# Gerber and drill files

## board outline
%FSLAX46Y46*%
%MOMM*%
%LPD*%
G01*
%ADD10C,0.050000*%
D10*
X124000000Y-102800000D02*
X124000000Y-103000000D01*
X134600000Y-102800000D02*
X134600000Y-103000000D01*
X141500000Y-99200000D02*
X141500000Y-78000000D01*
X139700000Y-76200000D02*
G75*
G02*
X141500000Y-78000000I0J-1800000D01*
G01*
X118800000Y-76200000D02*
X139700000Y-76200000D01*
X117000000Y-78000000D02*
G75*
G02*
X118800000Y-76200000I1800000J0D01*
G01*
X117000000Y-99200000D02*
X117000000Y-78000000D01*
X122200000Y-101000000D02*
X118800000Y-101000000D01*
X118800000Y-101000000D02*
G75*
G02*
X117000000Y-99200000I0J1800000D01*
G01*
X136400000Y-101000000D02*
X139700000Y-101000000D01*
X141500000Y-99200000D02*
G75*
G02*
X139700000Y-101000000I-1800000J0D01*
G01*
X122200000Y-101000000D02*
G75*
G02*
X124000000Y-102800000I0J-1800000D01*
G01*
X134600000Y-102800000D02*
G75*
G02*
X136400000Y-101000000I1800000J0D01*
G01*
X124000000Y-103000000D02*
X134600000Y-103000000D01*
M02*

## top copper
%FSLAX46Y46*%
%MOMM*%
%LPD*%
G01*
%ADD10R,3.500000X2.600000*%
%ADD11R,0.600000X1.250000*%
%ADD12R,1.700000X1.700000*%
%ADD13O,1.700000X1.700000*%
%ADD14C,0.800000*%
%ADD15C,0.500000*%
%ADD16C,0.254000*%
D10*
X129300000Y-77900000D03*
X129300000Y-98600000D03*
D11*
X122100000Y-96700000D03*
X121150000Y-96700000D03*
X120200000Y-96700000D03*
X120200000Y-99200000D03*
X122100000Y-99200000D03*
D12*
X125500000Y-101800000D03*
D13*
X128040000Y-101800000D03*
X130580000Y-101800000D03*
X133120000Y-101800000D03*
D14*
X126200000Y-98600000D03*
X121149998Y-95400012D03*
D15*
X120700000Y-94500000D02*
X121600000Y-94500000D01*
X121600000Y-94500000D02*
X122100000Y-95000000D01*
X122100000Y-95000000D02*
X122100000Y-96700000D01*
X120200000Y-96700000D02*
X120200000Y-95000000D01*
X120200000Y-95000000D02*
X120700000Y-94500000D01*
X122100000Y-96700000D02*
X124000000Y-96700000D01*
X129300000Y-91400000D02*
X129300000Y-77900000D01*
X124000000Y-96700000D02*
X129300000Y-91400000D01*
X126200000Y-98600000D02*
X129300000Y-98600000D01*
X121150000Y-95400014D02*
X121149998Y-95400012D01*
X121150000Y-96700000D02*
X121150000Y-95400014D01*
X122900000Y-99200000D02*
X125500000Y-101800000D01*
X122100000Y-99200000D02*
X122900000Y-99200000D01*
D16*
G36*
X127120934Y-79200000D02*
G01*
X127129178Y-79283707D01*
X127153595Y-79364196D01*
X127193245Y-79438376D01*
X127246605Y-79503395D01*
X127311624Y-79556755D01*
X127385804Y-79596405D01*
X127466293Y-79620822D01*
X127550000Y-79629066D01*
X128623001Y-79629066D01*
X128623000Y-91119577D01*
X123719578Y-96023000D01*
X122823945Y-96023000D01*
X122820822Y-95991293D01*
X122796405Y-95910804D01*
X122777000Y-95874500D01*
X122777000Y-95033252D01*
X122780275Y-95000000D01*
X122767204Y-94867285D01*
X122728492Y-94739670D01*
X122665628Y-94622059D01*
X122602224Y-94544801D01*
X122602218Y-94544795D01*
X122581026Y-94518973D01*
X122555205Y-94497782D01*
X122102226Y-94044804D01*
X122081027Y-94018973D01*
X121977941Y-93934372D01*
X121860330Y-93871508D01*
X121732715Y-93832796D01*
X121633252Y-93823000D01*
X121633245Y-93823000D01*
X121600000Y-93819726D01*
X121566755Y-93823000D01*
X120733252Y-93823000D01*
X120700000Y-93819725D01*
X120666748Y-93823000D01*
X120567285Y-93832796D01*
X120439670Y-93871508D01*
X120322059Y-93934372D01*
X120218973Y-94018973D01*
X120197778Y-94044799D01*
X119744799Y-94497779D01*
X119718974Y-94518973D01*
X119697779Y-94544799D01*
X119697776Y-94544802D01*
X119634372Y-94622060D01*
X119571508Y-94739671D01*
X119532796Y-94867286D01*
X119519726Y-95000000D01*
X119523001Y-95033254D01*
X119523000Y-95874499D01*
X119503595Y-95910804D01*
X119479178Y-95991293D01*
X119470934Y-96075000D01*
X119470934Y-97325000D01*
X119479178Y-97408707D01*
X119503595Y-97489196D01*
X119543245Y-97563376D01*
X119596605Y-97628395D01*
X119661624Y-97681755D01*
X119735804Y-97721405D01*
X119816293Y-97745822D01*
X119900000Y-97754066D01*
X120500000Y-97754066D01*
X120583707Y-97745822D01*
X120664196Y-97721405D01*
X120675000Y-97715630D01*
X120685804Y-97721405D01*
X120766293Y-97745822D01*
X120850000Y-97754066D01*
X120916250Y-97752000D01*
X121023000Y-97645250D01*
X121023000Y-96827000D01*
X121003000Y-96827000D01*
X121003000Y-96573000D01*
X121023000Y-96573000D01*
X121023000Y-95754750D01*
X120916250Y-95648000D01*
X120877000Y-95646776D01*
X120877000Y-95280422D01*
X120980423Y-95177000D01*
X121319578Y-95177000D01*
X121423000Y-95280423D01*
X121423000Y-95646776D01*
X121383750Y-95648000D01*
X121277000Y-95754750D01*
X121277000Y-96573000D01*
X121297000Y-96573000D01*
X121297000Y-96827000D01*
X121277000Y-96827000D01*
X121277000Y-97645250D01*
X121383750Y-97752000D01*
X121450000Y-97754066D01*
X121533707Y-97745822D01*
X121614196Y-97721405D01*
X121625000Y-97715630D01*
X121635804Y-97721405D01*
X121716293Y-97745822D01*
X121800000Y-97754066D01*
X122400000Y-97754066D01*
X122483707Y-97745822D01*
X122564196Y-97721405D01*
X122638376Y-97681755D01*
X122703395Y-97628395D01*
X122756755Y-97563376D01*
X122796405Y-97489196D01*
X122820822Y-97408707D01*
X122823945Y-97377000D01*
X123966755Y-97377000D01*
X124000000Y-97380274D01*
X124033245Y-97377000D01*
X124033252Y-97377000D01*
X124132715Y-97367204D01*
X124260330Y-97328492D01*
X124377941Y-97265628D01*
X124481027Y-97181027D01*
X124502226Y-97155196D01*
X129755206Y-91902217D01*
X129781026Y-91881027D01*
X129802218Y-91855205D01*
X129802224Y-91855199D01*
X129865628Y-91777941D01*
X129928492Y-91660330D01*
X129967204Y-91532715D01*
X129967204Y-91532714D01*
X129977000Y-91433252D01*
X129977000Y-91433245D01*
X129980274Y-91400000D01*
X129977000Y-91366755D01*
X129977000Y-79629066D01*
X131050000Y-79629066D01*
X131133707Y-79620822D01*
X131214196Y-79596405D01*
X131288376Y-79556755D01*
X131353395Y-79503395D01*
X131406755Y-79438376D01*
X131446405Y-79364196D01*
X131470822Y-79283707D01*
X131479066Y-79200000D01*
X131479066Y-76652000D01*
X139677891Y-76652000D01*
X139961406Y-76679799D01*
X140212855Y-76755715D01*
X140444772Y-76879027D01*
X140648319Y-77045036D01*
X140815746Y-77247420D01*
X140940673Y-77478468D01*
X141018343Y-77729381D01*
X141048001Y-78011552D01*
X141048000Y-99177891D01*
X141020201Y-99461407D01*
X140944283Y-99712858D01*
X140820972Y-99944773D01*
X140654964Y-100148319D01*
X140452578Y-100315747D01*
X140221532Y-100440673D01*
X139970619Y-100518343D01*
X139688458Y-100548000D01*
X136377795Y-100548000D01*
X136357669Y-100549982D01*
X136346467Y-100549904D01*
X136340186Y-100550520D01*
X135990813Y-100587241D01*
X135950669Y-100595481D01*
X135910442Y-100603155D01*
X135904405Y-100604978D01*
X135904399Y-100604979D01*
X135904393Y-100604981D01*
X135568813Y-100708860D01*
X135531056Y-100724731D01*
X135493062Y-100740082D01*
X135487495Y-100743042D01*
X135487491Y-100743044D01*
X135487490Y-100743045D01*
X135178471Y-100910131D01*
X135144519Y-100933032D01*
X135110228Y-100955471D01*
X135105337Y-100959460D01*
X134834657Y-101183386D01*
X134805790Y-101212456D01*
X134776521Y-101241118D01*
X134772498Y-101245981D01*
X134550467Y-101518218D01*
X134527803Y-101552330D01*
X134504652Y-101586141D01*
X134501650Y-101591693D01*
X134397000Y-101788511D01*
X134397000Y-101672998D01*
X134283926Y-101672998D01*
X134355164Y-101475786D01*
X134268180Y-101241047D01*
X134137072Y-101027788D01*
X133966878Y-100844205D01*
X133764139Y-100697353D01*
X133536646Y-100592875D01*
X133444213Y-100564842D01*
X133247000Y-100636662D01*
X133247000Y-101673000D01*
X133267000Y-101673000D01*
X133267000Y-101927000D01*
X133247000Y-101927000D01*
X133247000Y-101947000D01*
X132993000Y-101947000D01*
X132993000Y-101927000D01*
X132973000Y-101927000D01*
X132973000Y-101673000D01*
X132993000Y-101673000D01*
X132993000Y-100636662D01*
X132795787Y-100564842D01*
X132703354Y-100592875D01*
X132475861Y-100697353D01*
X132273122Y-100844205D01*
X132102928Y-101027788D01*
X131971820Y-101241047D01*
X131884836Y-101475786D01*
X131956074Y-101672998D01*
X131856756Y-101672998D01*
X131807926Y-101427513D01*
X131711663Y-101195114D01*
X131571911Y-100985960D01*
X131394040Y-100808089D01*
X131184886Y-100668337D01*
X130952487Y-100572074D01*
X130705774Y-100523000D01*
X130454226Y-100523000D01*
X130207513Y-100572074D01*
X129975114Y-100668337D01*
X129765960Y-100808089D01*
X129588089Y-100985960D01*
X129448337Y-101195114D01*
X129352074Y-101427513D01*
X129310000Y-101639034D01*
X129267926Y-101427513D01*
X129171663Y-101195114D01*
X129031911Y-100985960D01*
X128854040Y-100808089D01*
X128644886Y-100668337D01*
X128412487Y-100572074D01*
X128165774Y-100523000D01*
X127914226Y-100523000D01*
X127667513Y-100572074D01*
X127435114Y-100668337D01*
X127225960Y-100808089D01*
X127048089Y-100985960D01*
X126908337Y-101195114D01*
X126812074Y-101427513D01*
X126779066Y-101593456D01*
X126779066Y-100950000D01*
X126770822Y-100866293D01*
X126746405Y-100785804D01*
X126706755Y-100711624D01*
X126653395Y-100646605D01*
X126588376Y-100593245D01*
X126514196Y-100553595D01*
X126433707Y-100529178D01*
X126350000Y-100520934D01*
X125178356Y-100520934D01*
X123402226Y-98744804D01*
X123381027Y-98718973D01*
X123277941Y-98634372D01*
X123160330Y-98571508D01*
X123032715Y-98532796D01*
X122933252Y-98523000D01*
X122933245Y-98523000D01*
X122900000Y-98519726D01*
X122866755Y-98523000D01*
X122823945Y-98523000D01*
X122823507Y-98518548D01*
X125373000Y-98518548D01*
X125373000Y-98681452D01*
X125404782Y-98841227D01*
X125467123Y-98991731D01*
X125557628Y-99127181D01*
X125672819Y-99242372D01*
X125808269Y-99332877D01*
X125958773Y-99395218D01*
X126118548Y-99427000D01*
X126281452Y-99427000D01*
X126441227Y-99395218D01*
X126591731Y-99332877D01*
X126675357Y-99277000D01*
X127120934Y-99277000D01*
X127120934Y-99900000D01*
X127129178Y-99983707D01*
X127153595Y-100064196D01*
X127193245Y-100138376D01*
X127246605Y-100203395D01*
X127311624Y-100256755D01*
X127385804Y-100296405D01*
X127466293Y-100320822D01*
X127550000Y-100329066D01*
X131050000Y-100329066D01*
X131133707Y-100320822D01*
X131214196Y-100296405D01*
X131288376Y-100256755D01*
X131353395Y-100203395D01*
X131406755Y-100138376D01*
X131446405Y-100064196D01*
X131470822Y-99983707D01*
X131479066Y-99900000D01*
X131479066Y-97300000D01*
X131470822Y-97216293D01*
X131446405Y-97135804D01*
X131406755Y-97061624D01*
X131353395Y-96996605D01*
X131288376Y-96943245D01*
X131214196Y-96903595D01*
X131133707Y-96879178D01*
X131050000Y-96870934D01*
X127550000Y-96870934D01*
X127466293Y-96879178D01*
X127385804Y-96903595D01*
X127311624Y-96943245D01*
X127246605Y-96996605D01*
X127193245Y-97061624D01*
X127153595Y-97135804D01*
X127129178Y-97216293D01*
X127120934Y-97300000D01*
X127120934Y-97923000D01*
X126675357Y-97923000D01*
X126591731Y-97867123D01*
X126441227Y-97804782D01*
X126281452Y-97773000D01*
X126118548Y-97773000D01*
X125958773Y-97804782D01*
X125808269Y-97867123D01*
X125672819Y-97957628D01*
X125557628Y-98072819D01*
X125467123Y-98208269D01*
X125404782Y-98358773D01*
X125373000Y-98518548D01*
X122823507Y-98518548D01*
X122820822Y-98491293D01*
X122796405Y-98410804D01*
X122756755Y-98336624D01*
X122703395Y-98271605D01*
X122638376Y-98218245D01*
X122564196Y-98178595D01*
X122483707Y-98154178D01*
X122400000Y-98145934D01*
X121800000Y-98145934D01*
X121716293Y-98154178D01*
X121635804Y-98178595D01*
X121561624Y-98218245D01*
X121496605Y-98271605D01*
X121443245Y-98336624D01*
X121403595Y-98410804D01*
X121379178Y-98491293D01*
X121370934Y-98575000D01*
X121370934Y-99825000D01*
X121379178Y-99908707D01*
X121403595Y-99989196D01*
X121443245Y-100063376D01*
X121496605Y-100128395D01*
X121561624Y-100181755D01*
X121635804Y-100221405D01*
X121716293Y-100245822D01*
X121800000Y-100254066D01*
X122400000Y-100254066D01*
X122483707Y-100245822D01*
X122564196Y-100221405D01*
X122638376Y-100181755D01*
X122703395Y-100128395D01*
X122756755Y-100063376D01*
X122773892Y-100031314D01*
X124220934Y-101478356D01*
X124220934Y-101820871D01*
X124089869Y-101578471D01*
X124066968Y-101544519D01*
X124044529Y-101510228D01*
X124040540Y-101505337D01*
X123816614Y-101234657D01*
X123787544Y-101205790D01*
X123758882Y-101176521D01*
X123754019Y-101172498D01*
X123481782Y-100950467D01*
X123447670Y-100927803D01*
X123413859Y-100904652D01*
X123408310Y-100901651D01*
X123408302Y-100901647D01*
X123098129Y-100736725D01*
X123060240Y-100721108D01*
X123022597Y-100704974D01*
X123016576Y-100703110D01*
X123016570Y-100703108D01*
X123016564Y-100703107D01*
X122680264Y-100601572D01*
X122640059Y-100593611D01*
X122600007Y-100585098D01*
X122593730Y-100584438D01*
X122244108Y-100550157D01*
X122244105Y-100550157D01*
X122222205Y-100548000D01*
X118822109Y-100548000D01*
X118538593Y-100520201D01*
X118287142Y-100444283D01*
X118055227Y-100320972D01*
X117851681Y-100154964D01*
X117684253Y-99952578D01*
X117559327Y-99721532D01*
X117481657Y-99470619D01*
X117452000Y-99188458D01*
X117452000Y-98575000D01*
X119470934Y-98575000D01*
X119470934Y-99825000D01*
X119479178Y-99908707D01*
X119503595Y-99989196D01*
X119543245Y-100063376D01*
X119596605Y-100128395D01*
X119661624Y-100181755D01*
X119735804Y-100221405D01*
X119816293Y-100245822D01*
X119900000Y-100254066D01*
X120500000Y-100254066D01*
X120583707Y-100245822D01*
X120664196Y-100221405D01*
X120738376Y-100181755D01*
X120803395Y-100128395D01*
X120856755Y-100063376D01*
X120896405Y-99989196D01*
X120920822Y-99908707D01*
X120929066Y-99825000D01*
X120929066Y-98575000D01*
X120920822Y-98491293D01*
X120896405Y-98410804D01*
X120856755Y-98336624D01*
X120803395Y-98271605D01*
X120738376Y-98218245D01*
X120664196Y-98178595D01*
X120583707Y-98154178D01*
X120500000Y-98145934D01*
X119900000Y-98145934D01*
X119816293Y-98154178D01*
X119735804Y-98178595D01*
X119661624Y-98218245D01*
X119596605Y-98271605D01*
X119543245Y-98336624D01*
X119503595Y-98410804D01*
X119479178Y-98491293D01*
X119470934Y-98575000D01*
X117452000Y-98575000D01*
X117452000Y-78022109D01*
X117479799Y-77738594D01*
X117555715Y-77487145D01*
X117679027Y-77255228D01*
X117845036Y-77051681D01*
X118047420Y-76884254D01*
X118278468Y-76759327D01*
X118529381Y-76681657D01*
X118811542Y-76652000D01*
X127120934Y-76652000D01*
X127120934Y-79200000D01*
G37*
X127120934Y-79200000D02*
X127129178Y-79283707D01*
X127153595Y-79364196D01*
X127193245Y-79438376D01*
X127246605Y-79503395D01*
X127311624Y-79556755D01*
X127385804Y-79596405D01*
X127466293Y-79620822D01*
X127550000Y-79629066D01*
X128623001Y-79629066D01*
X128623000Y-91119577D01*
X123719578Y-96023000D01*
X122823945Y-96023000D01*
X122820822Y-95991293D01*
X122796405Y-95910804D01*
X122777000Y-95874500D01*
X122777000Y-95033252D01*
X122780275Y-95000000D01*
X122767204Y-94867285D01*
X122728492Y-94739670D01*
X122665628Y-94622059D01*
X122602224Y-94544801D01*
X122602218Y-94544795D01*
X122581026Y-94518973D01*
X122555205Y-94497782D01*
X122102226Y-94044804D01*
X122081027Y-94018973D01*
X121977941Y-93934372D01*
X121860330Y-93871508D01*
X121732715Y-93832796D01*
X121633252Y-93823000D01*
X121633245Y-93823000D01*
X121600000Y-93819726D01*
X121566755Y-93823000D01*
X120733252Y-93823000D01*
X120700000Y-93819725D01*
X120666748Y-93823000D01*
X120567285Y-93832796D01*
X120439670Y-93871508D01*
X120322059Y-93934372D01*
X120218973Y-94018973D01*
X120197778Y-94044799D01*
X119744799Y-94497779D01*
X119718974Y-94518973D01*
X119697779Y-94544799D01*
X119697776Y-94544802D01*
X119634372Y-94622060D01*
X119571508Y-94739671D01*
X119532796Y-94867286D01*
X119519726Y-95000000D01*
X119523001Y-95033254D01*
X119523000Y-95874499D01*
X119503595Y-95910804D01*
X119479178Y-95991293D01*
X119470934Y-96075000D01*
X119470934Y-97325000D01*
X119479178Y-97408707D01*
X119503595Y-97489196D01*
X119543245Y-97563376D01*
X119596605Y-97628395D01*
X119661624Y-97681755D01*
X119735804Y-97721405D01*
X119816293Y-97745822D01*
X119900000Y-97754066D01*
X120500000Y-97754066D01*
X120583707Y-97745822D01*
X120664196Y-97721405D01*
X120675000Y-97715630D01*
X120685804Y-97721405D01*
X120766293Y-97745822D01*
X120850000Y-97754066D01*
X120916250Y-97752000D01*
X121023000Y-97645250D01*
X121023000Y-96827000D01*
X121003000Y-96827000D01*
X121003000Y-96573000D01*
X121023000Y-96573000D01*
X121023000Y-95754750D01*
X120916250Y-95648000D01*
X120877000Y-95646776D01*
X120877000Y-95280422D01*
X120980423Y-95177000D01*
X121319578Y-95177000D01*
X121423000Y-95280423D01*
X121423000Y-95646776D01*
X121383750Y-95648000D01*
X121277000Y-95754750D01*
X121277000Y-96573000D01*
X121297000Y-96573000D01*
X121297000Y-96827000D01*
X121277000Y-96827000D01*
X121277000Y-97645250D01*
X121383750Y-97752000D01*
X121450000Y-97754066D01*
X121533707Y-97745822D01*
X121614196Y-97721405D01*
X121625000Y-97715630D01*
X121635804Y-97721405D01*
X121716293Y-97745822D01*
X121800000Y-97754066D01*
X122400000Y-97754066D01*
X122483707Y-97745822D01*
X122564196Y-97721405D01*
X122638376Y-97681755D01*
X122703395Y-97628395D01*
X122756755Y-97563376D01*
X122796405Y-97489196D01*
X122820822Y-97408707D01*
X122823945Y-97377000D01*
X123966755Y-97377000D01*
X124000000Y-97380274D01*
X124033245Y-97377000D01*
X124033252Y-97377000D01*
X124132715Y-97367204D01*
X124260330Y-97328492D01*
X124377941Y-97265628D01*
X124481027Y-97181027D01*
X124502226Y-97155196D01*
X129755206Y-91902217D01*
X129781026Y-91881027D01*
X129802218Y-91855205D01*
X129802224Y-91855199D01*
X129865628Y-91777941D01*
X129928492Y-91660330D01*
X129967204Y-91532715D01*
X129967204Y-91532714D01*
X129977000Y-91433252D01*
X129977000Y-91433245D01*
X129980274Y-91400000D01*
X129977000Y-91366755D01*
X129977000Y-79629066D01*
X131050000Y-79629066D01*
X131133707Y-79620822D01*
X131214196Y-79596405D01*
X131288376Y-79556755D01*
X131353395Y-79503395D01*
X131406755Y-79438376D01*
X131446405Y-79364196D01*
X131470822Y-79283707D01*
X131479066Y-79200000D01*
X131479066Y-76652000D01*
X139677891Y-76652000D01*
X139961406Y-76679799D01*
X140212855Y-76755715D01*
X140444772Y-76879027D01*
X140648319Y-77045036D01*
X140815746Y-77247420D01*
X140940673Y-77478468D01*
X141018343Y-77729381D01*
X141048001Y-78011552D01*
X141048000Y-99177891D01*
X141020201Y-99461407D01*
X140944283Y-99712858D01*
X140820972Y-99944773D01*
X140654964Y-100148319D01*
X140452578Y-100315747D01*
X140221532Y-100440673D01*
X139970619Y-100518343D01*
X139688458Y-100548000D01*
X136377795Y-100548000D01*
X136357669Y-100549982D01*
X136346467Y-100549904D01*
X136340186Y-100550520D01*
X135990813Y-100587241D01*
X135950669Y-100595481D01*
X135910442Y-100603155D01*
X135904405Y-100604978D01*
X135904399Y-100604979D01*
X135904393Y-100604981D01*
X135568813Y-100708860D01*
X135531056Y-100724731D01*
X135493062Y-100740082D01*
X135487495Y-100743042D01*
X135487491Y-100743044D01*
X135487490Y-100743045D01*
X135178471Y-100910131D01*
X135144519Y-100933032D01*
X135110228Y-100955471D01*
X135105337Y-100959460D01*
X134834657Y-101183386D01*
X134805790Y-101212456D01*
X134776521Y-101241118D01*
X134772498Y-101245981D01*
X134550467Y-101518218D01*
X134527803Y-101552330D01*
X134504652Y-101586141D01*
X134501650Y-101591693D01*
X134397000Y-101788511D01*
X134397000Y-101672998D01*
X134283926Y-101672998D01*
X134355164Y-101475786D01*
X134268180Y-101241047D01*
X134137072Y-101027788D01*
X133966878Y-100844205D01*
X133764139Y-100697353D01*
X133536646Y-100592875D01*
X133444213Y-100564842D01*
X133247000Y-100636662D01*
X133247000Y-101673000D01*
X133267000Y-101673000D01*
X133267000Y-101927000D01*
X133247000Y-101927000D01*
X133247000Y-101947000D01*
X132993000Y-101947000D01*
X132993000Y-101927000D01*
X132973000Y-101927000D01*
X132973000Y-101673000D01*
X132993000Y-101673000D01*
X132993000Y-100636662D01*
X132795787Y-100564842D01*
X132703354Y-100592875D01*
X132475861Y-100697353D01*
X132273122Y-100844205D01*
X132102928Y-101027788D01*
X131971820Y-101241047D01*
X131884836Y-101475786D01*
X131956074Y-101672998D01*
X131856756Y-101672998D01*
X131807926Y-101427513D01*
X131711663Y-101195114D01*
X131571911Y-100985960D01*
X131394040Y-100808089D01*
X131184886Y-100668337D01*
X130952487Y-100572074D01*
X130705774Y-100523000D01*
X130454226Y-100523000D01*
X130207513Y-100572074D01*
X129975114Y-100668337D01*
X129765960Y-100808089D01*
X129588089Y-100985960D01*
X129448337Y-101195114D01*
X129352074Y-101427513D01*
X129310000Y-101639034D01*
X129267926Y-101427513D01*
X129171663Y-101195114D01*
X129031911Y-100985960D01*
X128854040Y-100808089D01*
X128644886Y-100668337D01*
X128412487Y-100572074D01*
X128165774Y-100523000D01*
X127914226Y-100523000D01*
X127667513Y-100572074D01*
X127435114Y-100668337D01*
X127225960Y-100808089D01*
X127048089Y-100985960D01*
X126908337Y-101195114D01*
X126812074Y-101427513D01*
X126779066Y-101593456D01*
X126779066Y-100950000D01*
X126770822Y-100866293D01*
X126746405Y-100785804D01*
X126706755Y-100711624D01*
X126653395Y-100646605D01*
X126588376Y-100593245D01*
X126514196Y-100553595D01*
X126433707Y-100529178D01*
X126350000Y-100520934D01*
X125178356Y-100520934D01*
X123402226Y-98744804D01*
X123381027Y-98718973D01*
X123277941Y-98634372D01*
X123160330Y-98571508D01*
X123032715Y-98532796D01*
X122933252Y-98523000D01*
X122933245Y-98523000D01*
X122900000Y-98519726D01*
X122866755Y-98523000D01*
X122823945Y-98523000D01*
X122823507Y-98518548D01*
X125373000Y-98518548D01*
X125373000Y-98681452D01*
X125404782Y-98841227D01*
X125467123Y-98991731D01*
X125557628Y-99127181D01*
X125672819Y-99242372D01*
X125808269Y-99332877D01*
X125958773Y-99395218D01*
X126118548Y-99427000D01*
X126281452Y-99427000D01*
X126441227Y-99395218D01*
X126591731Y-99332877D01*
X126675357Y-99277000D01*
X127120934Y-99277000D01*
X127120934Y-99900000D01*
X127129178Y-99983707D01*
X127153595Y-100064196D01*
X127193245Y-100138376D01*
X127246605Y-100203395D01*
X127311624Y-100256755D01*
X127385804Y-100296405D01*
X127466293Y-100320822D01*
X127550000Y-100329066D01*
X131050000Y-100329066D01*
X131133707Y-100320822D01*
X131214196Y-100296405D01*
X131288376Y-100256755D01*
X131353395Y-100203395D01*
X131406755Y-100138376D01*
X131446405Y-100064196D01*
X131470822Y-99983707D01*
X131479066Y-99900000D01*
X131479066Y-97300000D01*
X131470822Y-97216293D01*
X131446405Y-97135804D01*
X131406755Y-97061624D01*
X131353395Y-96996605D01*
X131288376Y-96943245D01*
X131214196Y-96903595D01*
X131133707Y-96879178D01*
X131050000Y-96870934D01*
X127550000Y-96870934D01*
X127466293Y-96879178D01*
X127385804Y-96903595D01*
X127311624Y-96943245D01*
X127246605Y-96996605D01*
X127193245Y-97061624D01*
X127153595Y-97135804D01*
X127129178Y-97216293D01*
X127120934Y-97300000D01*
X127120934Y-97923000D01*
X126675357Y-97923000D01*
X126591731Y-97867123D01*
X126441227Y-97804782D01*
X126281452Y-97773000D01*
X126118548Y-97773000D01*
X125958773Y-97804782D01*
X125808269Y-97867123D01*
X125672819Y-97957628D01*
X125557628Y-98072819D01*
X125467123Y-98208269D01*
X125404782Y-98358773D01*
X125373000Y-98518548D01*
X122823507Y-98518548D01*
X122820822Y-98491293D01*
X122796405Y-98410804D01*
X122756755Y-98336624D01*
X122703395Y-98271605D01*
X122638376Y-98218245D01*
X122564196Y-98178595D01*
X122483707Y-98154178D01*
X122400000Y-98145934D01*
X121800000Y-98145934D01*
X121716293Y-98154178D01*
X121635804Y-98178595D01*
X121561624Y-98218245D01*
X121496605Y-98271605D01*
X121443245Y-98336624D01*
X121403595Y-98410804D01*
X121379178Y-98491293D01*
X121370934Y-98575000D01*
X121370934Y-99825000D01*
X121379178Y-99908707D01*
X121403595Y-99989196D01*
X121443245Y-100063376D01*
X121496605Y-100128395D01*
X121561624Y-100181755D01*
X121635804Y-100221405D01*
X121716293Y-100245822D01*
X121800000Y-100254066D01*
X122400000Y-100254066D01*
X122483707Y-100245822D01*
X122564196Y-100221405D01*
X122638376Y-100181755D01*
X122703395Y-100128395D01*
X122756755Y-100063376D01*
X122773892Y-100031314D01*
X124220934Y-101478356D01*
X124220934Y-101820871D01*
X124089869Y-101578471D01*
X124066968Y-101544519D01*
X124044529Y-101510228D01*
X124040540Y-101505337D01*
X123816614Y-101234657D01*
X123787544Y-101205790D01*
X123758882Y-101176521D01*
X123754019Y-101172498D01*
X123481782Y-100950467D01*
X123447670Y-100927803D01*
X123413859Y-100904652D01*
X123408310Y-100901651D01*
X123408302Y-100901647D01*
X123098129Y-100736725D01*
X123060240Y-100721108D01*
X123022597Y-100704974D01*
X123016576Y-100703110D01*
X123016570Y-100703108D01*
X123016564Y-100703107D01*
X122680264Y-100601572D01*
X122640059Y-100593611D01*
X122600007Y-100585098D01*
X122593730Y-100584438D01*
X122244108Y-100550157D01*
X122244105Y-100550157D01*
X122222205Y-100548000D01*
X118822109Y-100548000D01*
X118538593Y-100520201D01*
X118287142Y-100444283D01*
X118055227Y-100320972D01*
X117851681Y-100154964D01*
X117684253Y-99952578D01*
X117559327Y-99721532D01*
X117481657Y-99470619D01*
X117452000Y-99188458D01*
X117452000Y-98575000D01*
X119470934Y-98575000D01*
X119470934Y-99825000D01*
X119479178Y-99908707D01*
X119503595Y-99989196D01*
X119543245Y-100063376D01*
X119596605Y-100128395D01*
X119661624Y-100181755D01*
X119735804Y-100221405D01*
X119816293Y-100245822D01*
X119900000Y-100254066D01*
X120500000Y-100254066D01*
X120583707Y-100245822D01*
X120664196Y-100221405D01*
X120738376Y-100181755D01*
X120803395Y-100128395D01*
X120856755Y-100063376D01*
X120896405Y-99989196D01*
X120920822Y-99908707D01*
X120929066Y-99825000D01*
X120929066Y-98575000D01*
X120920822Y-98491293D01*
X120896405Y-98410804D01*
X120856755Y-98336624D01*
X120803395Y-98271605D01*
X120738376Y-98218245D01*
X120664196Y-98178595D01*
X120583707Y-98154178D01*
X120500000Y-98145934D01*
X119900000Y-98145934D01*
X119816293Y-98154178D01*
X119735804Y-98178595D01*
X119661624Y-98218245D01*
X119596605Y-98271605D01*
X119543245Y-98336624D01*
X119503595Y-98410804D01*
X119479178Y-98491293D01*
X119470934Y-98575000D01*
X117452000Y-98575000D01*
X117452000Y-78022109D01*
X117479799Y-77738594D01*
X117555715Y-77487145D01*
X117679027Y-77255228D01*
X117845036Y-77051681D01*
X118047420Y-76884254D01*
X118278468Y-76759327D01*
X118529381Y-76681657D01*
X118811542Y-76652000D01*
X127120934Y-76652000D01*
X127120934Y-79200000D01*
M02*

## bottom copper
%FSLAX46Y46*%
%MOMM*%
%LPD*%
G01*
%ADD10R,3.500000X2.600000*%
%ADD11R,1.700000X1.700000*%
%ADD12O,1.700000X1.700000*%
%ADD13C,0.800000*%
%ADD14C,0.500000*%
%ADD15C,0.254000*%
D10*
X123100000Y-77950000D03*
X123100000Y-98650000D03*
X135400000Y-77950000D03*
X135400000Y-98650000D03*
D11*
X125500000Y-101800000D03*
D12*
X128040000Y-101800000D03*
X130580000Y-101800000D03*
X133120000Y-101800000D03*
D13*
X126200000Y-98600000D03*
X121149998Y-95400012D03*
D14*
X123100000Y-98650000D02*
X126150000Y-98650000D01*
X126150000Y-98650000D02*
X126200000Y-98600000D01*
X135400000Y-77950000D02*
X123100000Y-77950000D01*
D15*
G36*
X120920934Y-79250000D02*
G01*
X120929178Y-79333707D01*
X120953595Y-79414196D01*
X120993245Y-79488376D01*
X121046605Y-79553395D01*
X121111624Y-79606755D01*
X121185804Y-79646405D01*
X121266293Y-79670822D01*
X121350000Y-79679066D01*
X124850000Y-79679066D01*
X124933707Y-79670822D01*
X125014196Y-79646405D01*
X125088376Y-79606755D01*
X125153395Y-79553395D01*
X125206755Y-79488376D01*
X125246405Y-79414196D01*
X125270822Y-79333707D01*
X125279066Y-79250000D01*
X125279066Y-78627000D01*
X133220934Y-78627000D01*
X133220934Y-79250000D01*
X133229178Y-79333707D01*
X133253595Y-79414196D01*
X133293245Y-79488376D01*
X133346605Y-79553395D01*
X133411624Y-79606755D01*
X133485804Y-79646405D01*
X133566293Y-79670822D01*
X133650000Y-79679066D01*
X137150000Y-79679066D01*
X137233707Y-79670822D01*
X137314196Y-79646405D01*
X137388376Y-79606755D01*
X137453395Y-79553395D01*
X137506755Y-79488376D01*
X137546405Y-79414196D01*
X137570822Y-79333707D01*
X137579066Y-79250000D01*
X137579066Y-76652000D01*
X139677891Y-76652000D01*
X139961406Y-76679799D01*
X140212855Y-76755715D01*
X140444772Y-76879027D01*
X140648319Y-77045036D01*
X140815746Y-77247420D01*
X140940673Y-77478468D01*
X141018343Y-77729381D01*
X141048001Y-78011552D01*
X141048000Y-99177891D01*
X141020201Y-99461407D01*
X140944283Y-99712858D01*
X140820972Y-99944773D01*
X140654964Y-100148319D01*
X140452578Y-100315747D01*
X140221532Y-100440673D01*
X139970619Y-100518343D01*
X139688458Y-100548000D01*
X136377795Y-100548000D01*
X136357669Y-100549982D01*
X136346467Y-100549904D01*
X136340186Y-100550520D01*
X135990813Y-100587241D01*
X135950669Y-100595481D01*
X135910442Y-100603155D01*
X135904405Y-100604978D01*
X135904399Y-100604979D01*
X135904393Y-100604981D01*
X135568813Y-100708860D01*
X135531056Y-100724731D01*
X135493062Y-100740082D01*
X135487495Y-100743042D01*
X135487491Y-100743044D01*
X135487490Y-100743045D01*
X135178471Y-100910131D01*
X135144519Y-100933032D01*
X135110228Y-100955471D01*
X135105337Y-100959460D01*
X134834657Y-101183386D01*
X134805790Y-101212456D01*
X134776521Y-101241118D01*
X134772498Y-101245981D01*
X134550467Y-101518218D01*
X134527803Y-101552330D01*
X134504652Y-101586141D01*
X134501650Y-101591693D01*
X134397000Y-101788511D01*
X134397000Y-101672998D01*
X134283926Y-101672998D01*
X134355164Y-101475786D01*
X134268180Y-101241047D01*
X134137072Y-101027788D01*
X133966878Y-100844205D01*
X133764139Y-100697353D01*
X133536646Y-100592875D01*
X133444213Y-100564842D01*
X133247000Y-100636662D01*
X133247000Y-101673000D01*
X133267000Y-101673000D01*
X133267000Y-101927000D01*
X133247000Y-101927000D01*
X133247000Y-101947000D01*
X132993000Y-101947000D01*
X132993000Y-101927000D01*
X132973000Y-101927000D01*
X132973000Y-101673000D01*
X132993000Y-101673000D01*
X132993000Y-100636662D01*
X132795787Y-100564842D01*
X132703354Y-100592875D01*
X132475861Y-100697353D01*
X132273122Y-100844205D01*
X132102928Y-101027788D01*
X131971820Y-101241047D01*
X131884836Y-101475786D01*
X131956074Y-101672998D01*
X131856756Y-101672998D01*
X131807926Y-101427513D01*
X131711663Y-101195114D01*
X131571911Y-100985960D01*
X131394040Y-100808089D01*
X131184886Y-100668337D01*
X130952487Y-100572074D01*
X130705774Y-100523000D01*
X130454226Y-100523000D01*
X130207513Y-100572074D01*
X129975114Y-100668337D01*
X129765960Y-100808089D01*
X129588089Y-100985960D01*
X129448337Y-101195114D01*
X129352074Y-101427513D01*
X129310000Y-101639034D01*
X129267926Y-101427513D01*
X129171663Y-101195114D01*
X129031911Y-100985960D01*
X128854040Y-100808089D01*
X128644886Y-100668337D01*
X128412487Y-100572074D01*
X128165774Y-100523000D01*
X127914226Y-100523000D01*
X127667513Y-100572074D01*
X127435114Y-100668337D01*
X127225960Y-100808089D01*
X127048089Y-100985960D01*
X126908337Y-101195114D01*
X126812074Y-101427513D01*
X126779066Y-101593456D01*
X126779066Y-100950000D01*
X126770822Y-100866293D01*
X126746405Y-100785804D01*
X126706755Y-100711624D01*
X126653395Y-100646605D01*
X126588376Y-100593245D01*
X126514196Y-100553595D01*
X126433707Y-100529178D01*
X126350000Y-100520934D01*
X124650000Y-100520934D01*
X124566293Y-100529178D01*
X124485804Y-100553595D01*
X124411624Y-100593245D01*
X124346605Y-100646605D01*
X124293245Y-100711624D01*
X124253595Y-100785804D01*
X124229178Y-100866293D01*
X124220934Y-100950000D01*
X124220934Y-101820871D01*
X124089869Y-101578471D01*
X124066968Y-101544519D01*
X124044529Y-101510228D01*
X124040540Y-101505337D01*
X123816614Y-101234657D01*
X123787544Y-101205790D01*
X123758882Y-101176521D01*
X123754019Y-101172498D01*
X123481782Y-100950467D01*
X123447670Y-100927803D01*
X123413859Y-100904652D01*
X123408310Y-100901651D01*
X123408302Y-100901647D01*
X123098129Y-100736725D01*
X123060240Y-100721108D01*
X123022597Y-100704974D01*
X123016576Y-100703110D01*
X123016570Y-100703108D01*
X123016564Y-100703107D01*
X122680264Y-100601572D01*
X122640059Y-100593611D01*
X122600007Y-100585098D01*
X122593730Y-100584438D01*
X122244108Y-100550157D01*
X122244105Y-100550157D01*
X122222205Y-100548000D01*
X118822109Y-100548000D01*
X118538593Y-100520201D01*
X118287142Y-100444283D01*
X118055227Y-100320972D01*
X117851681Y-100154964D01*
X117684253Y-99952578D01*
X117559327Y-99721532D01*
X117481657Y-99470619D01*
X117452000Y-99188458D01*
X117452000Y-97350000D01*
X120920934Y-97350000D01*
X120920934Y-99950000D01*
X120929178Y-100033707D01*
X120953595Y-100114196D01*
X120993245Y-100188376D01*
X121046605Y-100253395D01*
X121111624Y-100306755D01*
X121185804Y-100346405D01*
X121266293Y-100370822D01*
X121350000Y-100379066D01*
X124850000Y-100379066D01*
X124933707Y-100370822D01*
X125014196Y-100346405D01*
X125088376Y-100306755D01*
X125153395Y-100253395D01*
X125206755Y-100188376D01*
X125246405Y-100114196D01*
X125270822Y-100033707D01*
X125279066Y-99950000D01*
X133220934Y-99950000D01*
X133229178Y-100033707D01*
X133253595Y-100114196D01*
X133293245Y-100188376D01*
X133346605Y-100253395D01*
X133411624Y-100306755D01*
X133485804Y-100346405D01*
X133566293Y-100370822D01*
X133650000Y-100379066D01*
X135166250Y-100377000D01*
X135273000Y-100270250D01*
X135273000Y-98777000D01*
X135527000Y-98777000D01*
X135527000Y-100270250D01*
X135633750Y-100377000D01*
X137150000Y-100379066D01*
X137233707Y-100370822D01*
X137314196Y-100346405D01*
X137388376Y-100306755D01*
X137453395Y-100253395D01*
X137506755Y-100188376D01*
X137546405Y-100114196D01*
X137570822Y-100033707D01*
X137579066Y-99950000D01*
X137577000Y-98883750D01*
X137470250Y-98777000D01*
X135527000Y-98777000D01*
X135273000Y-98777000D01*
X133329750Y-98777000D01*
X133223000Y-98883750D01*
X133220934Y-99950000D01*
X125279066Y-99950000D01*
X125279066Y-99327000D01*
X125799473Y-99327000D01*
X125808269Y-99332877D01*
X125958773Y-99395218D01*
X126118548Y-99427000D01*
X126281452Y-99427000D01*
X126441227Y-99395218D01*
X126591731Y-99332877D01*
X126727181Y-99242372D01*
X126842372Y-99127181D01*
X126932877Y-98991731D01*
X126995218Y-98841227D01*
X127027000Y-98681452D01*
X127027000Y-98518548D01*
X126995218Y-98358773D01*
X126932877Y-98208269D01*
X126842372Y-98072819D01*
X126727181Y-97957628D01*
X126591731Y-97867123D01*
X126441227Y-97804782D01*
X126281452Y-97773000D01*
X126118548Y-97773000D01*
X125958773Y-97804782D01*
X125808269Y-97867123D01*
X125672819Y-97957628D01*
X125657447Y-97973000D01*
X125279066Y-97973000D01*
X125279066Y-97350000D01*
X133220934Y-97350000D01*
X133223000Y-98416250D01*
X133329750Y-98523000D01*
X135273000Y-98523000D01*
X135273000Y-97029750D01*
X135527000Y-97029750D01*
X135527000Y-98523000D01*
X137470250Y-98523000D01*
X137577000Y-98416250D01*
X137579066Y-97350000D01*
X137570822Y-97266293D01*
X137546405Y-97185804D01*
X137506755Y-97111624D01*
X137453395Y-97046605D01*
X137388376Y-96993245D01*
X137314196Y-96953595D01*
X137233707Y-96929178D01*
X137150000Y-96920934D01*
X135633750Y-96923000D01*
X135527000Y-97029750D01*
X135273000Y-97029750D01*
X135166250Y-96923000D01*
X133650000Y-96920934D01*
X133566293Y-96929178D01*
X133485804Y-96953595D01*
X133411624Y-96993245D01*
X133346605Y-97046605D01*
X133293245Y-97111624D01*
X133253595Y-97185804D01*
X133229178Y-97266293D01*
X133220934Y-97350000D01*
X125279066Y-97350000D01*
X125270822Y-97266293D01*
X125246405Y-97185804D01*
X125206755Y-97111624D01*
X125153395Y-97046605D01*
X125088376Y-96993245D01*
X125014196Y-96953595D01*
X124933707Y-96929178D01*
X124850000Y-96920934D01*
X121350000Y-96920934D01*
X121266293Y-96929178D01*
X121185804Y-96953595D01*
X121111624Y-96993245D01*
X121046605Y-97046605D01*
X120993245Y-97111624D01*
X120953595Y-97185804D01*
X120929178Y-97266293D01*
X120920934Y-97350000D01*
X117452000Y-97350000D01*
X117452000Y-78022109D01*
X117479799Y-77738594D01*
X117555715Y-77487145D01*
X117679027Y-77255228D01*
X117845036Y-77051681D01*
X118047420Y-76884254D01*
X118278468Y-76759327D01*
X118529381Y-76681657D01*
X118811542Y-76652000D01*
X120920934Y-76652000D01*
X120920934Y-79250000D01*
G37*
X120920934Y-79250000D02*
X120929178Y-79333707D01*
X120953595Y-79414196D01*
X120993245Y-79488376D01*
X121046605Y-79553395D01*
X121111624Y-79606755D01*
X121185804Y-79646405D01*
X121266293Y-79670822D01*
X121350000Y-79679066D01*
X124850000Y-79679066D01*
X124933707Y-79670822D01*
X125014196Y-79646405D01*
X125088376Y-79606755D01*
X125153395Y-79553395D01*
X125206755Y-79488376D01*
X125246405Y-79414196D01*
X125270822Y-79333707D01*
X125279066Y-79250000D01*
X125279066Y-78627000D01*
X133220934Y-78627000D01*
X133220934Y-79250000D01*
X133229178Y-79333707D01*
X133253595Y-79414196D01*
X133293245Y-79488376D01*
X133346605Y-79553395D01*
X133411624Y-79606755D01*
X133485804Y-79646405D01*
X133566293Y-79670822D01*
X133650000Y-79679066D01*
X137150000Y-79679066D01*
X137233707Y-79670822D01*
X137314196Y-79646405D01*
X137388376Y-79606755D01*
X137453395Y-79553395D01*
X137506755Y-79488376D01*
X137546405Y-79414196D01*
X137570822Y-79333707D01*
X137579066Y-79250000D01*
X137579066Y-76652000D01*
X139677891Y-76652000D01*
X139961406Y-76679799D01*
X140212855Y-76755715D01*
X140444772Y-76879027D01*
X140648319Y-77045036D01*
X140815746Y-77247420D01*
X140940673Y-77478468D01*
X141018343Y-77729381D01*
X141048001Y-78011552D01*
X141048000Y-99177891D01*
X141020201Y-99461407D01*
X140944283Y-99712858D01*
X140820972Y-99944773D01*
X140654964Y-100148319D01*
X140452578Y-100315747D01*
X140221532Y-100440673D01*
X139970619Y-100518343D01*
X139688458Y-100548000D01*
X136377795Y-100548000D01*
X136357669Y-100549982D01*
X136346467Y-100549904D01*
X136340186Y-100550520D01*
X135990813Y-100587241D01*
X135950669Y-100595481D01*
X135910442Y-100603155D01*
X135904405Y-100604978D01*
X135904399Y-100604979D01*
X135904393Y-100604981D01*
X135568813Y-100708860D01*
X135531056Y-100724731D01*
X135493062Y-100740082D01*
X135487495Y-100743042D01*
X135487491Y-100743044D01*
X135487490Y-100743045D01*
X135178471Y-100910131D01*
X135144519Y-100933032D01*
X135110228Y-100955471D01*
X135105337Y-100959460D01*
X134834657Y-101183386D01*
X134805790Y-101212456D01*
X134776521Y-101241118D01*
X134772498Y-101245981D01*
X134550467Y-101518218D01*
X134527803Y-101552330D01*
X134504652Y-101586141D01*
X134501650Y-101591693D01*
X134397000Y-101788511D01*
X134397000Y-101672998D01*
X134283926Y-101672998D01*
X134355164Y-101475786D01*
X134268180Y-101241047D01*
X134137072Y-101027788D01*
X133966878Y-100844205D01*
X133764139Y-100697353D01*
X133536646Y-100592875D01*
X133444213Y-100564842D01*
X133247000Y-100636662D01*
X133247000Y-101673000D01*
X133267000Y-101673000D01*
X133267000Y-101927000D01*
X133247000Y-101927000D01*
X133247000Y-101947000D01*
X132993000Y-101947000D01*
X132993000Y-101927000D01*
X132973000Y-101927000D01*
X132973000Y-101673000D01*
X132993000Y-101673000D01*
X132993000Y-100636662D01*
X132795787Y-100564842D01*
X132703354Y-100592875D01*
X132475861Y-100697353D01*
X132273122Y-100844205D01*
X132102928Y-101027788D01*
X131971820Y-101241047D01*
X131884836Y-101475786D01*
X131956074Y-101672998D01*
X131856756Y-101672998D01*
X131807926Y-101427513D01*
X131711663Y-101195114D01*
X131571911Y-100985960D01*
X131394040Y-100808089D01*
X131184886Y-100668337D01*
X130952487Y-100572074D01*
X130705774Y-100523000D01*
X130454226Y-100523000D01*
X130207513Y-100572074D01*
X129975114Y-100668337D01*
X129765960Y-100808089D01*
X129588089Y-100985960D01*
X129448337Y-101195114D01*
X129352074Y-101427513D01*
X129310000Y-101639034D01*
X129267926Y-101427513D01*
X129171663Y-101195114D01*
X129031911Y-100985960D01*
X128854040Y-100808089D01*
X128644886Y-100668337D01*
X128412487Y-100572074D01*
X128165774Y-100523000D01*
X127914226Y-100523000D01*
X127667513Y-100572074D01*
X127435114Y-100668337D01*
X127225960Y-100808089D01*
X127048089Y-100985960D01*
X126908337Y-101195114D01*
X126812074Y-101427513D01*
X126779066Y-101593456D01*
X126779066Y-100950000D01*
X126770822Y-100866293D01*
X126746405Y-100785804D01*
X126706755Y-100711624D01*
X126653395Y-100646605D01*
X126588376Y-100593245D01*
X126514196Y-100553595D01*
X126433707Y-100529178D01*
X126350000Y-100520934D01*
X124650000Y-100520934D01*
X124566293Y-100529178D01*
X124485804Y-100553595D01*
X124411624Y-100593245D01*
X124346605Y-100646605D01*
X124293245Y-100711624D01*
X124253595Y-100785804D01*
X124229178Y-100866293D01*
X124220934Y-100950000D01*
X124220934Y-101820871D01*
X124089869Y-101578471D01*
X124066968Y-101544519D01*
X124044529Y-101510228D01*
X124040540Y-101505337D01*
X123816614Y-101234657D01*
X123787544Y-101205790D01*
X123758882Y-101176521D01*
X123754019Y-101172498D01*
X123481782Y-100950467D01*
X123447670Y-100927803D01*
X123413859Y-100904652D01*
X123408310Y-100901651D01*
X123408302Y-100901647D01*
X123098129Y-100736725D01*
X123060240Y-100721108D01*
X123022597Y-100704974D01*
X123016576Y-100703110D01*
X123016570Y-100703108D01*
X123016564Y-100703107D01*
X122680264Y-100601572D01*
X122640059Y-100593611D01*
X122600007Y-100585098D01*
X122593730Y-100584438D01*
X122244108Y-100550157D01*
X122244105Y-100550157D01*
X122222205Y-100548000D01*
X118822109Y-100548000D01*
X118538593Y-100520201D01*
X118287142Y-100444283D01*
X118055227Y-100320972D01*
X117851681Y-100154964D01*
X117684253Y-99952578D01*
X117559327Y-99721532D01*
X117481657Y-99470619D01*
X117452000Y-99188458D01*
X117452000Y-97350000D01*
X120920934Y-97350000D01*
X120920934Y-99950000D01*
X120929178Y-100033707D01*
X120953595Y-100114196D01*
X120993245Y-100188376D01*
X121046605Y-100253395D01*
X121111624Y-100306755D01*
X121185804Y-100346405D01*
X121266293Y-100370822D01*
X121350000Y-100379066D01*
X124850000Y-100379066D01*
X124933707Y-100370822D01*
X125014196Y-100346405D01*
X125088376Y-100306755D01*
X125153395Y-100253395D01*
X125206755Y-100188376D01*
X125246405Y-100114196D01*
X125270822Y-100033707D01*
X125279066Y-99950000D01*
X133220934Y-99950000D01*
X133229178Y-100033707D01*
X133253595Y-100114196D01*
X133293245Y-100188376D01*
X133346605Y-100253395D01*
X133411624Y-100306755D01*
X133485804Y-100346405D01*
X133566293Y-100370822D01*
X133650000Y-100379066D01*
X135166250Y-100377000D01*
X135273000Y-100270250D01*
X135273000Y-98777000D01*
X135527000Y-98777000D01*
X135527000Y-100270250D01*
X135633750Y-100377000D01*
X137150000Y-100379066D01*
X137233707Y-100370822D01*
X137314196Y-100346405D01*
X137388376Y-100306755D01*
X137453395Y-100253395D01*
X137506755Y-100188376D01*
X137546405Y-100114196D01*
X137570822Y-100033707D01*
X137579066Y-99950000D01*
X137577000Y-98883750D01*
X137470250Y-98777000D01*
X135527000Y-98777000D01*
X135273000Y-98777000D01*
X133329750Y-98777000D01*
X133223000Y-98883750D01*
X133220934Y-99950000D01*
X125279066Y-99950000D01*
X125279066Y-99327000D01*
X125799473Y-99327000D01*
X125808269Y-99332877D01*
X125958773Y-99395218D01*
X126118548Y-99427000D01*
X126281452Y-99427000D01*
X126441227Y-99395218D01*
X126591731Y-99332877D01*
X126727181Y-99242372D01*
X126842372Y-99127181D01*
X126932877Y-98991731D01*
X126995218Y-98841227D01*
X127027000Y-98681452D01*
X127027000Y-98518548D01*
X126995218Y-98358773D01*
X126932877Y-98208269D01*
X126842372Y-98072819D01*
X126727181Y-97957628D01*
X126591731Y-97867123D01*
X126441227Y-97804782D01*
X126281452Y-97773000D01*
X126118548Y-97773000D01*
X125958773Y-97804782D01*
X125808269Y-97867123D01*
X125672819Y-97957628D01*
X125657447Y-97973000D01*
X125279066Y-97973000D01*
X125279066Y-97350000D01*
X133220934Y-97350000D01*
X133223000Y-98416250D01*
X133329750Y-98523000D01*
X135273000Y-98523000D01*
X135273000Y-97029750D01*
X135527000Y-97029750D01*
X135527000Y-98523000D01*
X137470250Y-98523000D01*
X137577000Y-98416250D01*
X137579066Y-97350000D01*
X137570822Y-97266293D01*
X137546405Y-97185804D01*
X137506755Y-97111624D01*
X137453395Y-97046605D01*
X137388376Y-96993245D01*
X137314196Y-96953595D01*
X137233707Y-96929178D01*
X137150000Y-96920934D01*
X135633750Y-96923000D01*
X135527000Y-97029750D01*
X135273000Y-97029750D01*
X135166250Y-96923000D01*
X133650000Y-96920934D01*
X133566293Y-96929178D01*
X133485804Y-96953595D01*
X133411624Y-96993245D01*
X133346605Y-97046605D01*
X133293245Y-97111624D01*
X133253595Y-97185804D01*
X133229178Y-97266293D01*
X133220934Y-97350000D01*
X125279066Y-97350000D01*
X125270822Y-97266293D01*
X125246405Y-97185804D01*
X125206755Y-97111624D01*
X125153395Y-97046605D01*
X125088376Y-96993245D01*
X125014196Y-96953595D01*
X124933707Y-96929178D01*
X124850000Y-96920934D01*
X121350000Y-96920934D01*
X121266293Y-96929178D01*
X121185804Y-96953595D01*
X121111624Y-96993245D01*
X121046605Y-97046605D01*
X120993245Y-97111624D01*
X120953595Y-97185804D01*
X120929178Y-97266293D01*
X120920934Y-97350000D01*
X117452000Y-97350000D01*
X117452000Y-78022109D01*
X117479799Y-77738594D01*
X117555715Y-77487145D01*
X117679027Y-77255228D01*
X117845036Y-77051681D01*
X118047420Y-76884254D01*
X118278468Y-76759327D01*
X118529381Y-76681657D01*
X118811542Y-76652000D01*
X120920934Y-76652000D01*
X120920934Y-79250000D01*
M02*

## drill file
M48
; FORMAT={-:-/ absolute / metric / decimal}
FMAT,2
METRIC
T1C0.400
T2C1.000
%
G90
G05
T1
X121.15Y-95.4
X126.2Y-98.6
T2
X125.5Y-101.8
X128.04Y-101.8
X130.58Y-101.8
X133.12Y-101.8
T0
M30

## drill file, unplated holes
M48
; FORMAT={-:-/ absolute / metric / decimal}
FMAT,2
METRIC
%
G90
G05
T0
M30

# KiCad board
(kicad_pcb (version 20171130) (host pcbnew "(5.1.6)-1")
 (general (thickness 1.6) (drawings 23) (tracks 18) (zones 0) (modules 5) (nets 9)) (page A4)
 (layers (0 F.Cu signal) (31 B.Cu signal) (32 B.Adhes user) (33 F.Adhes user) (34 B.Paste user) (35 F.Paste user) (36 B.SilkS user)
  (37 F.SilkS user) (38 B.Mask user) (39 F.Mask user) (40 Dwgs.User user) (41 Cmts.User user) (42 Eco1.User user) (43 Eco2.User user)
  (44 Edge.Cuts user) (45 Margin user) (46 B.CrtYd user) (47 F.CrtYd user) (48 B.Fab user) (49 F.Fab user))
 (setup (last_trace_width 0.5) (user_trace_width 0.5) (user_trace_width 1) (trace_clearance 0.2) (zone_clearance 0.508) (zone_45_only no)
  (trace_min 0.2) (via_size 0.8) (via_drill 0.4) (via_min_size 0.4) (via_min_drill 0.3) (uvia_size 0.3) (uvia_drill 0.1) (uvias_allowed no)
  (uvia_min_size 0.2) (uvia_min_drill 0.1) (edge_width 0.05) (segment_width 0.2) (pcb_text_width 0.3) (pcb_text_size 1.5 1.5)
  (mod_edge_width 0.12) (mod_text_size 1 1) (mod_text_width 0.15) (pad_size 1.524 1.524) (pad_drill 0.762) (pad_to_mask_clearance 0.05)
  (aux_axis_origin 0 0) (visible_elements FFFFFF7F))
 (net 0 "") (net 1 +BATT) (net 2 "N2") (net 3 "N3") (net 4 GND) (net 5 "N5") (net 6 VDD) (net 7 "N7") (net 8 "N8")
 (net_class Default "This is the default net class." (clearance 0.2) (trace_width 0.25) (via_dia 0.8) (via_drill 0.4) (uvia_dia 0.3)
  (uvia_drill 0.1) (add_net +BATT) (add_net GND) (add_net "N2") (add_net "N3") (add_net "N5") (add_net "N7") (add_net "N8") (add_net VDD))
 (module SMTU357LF (layer F.Cu) (at 129.3 88.25 270)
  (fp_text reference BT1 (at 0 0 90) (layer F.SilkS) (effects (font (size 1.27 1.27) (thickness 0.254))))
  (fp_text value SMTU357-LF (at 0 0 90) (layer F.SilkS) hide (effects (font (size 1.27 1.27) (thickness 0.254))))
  (pad 1 smd rect (at -10.35 0 270) (size 2.6 3.5) (layers F.Cu F.Paste F.Mask) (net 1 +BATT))
  (pad 2 smd rect (at 10.35 0 270) (size 2.6 3.5) (layers F.Cu F.Paste F.Mask) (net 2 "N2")))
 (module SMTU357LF (layer B.Cu) (at 123.1 88.3 90)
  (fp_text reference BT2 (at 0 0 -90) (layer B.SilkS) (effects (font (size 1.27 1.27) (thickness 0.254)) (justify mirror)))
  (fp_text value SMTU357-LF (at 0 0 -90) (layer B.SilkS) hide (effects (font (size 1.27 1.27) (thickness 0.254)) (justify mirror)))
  (pad 2 smd rect (at 10.35 0 90) (size 2.6 3.5) (layers B.Cu B.Paste B.Mask) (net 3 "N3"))
  (pad 1 smd rect (at -10.35 0 90) (size 2.6 3.5) (layers B.Cu B.Paste B.Mask) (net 2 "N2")))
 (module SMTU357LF (layer B.Cu) (at 135.4 88.3 270)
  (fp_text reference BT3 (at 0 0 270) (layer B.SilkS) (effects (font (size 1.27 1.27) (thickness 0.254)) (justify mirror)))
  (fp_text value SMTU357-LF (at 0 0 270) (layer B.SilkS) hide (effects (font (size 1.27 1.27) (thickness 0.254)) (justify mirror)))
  (pad 1 smd rect (at -10.35 0 270) (size 2.6 3.5) (layers B.Cu B.Paste B.Mask) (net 3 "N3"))
  (pad 2 smd rect (at 10.35 0 270) (size 2.6 3.5) (layers B.Cu B.Paste B.Mask) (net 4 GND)))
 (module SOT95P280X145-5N (layer F.Cu) (at 121.15 97.95 270)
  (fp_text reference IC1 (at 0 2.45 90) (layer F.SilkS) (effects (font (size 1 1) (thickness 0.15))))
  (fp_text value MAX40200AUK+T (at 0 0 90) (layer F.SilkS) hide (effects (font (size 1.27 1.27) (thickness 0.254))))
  (pad 1 smd rect (at -1.25 -0.95) (size 0.6 1.25) (layers F.Cu F.Paste F.Mask) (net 1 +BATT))
  (pad 2 smd rect (at -1.25 0) (size 0.6 1.25) (layers F.Cu F.Paste F.Mask) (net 4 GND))
  (pad 3 smd rect (at -1.25 0.95) (size 0.6 1.25) (layers F.Cu F.Paste F.Mask) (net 1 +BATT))
  (pad 4 smd rect (at 1.25 0.95) (size 0.6 1.25) (layers F.Cu F.Paste F.Mask) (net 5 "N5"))
  (pad 5 smd rect (at 1.25 -0.95) (size 0.6 1.25) (layers F.Cu F.Paste F.Mask) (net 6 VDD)))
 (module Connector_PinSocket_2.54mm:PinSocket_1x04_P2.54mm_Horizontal (layer F.Cu) (at 125.5 101.8 90)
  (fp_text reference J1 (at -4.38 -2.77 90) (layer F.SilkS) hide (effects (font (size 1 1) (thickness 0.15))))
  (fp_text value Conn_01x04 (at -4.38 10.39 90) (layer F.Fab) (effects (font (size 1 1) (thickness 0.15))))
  (pad 1 thru_hole rect (at 0 0 90) (size 1.7 1.7) (drill 1) (layers *.Cu *.Mask) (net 6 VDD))
  (pad 2 thru_hole oval (at 0 2.54 90) (size 1.7 1.7) (drill 1) (layers *.Cu *.Mask) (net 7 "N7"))
  (pad 3 thru_hole oval (at 0 5.08 90) (size 1.7 1.7) (drill 1) (layers *.Cu *.Mask) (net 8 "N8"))
  (pad 4 thru_hole oval (at 0 7.62 90) (size 1.7 1.7) (drill 1) (layers *.Cu *.Mask) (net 4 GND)))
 (gr_line (start 124 102.8) (end 124 103) (layer Edge.Cuts) (width 0.05))
 (gr_line (start 134.6 102.8) (end 134.6 103) (layer Edge.Cuts) (width 0.05))
 (gr_line (start 141.5 99.2) (end 141.5 78) (layer Edge.Cuts) (width 0.05))
 (gr_arc (start 139.7 78) (end 141.5 78) (angle -90) (layer Edge.Cuts) (width 0.05))
 (gr_line (start 118.8 76.2) (end 139.7 76.2) (layer Edge.Cuts) (width 0.05))
 (gr_arc (start 118.8 78) (end 118.8 76.2) (angle -90) (layer Edge.Cuts) (width 0.05))
 (gr_line (start 117 99.2) (end 117 78) (layer Edge.Cuts) (width 0.05))
 (gr_line (start 122.2 101) (end 118.8 101) (layer Edge.Cuts) (width 0.05))
 (gr_arc (start 118.8 99.2) (end 117 99.2) (angle -90) (layer Edge.Cuts) (width 0.05))
 (gr_line (start 136.4 101) (end 139.7 101) (layer Edge.Cuts) (width 0.05))
 (gr_arc (start 139.7 99.2) (end 139.7 101) (angle -90) (layer Edge.Cuts) (width 0.05))
 (gr_arc (start 122.2 102.8) (end 124 102.8) (angle -90) (layer Edge.Cuts) (width 0.05))
 (gr_arc (start 136.4 102.8) (end 136.4 101) (angle -90) (layer Edge.Cuts) (width 0.05))
 (gr_line (start 124 103) (end 134.6 103) (layer Edge.Cuts) (width 0.05))
 (segment (start 120.7 94.5) (end 121.6 94.5) (width 0.5) (layer F.Cu) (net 1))
 (segment (start 121.6 94.5) (end 122.1 95) (width 0.5) (layer F.Cu) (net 1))
 (segment (start 122.1 95) (end 122.1 96.7) (width 0.5) (layer F.Cu) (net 1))
 (segment (start 120.2 96.7) (end 120.2 95) (width 0.5) (layer F.Cu) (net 1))
 (segment (start 120.2 95) (end 120.7 94.5) (width 0.5) (layer F.Cu) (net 1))
 (segment (start 122.1 96.7) (end 124 96.7) (width 0.5) (layer F.Cu) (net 1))
 (segment (start 129.3 91.4) (end 129.3 77.9) (width 0.5) (layer F.Cu) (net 1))
 (segment (start 124 96.7) (end 129.3 91.4) (width 0.5) (layer F.Cu) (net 1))
 (segment (start 123.1 98.65) (end 126.15 98.65) (width 0.5) (layer B.Cu) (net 2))
 (via (at 126.2 98.6) (size 0.8) (drill 0.4) (layers F.Cu B.Cu) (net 2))
 (segment (start 126.15 98.65) (end 126.2 98.6) (width 0.5) (layer B.Cu) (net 2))
 (segment (start 126.2 98.6) (end 129.3 98.6) (width 0.5) (layer F.Cu) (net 2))
 (segment (start 135.4 77.95) (end 123.1 77.95) (width 0.5) (layer B.Cu) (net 3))
 (via (at 121.149998 95.400012) (size 0.8) (drill 0.4) (layers F.Cu B.Cu) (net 4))
 (segment (start 121.15 95.400014) (end 121.149998 95.400012) (width 0.5) (layer F.Cu) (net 4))
 (segment (start 121.15 96.7) (end 121.15 95.400014) (width 0.5) (layer F.Cu) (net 4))
 (segment (start 122.9 99.2) (end 125.5 101.8) (width 0.5) (layer F.Cu) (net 6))
 (segment (start 122.1 99.2) (end 122.9 99.2) (width 0.5) (layer F.Cu) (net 6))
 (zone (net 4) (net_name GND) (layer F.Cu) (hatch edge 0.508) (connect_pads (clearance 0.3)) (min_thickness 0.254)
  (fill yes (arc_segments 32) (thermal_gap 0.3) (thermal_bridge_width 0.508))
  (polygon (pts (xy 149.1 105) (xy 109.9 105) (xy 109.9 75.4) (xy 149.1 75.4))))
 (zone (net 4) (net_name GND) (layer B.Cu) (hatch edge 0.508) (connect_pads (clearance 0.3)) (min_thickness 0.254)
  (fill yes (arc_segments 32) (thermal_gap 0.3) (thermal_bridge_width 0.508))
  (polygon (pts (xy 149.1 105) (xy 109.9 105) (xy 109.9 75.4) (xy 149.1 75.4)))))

